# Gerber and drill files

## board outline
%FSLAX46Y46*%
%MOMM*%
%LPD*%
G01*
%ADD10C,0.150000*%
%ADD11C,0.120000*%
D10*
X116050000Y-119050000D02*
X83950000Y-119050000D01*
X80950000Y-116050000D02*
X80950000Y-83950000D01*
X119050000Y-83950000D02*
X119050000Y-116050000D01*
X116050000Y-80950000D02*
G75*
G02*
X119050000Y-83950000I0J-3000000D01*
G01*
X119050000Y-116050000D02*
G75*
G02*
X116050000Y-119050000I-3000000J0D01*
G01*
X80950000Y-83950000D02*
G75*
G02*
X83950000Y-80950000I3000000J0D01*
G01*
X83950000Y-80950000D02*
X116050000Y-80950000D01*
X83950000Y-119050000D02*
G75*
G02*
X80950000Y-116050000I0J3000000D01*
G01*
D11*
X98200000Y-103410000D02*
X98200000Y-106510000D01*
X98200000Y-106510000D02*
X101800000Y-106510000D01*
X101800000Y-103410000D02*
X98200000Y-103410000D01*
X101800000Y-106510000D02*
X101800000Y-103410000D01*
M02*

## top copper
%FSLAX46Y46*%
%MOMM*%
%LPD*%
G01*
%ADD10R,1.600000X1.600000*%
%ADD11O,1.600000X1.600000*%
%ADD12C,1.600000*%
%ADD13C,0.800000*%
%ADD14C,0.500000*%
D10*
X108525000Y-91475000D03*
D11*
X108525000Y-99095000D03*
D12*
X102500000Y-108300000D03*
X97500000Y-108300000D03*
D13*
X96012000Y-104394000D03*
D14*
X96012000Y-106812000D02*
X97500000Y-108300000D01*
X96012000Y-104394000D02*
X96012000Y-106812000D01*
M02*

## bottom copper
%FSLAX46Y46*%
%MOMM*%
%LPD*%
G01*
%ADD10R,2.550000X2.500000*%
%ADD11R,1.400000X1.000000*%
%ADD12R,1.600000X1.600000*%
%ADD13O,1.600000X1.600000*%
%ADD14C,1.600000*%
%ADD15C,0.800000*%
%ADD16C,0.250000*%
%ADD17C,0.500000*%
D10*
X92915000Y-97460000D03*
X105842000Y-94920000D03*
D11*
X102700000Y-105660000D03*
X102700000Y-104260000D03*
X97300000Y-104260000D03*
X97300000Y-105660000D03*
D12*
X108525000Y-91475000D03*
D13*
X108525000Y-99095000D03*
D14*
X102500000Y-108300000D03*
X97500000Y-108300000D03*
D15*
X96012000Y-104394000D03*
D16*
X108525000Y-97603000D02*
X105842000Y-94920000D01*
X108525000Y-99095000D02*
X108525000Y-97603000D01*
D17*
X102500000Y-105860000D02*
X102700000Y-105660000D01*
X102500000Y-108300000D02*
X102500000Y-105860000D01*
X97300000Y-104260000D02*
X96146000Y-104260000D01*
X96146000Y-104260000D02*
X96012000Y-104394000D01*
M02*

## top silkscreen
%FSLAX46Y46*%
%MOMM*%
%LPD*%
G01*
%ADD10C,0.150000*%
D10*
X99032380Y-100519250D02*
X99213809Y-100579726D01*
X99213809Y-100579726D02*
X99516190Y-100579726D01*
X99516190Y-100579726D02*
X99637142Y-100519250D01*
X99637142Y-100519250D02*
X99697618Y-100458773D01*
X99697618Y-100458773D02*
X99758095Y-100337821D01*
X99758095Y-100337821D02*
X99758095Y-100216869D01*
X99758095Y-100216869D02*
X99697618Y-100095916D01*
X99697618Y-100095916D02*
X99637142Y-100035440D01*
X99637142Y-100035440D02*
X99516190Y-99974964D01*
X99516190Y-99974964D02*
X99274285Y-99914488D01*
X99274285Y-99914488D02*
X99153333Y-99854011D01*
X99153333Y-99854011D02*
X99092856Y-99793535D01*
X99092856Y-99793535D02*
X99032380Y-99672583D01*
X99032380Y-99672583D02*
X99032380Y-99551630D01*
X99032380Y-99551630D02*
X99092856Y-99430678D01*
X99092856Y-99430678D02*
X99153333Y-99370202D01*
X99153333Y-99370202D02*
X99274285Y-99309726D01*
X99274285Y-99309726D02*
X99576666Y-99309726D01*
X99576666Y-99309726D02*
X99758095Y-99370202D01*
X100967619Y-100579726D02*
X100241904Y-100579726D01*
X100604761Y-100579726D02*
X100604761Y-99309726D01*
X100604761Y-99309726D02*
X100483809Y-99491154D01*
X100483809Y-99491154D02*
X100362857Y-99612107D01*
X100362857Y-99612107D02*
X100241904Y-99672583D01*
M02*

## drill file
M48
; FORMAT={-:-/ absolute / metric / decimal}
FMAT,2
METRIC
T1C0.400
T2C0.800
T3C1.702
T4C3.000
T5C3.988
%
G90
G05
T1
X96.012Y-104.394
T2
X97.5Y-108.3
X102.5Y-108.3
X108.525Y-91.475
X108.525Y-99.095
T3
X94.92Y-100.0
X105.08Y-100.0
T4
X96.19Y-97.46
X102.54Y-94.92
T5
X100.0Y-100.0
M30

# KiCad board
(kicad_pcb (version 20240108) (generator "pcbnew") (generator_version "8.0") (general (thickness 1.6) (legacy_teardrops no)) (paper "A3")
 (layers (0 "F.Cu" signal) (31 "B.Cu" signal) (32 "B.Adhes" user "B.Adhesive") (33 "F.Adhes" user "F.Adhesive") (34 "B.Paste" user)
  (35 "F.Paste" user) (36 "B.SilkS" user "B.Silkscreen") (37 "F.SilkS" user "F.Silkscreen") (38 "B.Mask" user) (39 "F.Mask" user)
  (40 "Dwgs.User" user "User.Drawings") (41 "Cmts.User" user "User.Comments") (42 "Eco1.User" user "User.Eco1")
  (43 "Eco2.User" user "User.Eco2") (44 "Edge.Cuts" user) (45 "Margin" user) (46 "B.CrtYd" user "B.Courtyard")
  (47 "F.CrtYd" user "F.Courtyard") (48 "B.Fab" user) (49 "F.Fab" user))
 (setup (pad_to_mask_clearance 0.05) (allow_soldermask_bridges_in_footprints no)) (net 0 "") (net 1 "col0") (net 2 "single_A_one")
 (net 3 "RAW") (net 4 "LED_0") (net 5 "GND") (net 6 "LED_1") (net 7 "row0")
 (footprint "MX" (layer "F.Cu") (at 100 100)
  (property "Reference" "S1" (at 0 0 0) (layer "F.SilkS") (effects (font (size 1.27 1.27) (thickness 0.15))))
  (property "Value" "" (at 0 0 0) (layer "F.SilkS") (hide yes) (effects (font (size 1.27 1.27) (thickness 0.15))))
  (pad "" np_thru_hole circle (at -5.08 0) (size 1.7018 1.7018) (drill 1.7018) (layers "*.Cu" "*.Mask"))
  (pad "" np_thru_hole circle (at -3.81 -2.54) (size 3 3) (drill 3) (layers "*.Cu" "*.Mask"))
  (pad "" np_thru_hole circle (at 0 0) (size 3.9878 3.9878) (drill 3.9878) (layers "*.Cu" "*.Mask"))
  (pad "" np_thru_hole circle (at 2.54 -5.08) (size 3 3) (drill 3) (layers "*.Cu" "*.Mask"))
  (pad "" np_thru_hole circle (at 5.08 0) (size 1.7018 1.7018) (drill 1.7018) (layers "*.Cu" "*.Mask"))
  (pad "1" smd rect (at -7.085 -2.54) (size 2.55 2.5) (layers "B.Cu" "B.Paste" "B.Mask") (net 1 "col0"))
  (pad "2" smd rect (at 5.842 -5.08) (size 2.55 2.5) (layers "B.Cu" "B.Paste" "B.Mask") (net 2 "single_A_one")))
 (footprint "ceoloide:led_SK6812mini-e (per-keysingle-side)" (layer "B.Cu") (at 100 104.96)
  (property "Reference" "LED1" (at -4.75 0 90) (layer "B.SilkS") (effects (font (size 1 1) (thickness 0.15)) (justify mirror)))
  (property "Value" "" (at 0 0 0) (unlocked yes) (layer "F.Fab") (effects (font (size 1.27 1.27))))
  (fp_line (start -1.8 -1.55) (end -1.8 1.55) (stroke (width 0.12) (type solid)) (layer "Edge.Cuts"))
  (fp_line (start -1.8 1.55) (end 1.8 1.55) (stroke (width 0.12) (type solid)) (layer "Edge.Cuts"))
  (fp_line (start 1.8 -1.55) (end -1.8 -1.55) (stroke (width 0.12) (type solid)) (layer "Edge.Cuts"))
  (fp_line (start 1.8 1.55) (end 1.8 -1.55) (stroke (width 0.12) (type solid)) (layer "Edge.Cuts"))
  (pad "1" smd rect (at 2.7 0.7) (size 1.4 1) (layers "B.Cu" "B.Paste" "B.Mask") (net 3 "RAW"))
  (pad "2" smd rect (at 2.7 -0.7) (size 1.4 1) (layers "B.Cu" "B.Paste" "B.Mask") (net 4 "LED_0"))
  (pad "3" smd rect (at -2.7 -0.7) (size 1.4 1) (layers "B.Cu" "B.Paste" "B.Mask") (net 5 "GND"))
  (pad "4" smd rect (at -2.7 0.7) (size 1.4 1) (layers "B.Cu" "B.Paste" "B.Mask") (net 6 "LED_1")))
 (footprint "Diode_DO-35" (layer "B.Cu") (at 108.525 91.475 -90)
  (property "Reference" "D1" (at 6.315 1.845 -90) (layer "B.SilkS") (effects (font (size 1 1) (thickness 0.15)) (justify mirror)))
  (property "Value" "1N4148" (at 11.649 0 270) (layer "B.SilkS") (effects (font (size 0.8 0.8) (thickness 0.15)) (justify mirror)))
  (pad "1" thru_hole rect (at 0 0 270) (size 1.6 1.6) (drill 0.8) (layers "*.Cu" "*.Mask") (remove_unused_layers no) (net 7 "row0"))
  (pad "2" thru_hole oval (at 7.62 0 270) (size 1.6 1.6) (drill 0.8) (layers "*.Cu" "*.Mask") (remove_unused_layers no)
   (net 2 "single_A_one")))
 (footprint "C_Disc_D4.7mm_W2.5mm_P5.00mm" (layer "B.Cu") (at 102.5 108.3 180)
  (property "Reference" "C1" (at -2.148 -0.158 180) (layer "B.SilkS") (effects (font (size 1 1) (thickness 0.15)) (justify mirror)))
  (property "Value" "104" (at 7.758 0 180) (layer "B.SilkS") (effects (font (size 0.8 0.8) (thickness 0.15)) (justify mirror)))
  (pad "1" thru_hole circle (at 0 0) (size 1.6 1.6) (drill 0.8) (layers "*.Cu" "*.Mask") (remove_unused_layers no) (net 3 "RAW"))
  (pad "2" thru_hole circle (at 5 0) (size 1.6 1.6) (drill 0.8) (layers "*.Cu" "*.Mask") (remove_unused_layers no) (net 5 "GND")))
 (gr_line (start 116.05 119.05) (end 83.95 119.05) (stroke (width 0.15) (type solid)) (layer "Edge.Cuts"))
 (gr_line (start 80.95 116.05) (end 80.95 83.95) (stroke (width 0.15) (type solid)) (layer "Edge.Cuts"))
 (gr_line (start 119.05 83.95) (end 119.05 116.05) (stroke (width 0.15) (type solid)) (layer "Edge.Cuts"))
 (gr_arc (start 116.05 80.95) (mid 118.17132 81.82868) (end 119.05 83.95) (stroke (width 0.15) (type solid)) (layer "Edge.Cuts"))
 (gr_arc (start 119.05 116.05) (mid 118.17132 118.17132) (end 116.05 119.05) (stroke (width 0.15) (type solid)) (layer "Edge.Cuts"))
 (gr_arc (start 80.95 83.95) (mid 81.82868 81.82868) (end 83.95 80.95) (stroke (width 0.15) (type solid)) (layer "Edge.Cuts"))
 (gr_line (start 83.95 80.95) (end 116.05 80.95) (stroke (width 0.15) (type solid)) (layer "Edge.Cuts"))
 (gr_arc (start 83.95 119.05) (mid 81.82868 118.17132) (end 80.95 116.05) (stroke (width 0.15) (type solid)) (layer "Edge.Cuts"))
 (segment (start 108.525 97.603) (end 105.842 94.92) (width 0.25) (layer "B.Cu") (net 2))
 (segment (start 108.525 99.095) (end 108.525 97.603) (width 0.25) (layer "B.Cu") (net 2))
 (segment (start 102.5 105.86) (end 102.7 105.66) (width 0.5) (layer "B.Cu") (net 3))
 (segment (start 102.5 108.3) (end 102.5 105.86) (width 0.5) (layer "B.Cu") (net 3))
 (segment (start 96.012 106.812) (end 97.5 108.3) (width 0.5) (layer "F.Cu") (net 5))
 (segment (start 96.012 104.394) (end 96.012 106.812) (width 0.5) (layer "F.Cu") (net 5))
 (via (at 96.012 104.394) (size 0.8) (drill 0.4) (layers "F.Cu" "B.Cu") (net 5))
 (segment (start 97.3 104.26) (end 96.146 104.26) (width 0.5) (layer "B.Cu") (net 5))
 (segment (start 96.146 104.26) (end 96.012 104.394) (width 0.5) (layer "B.Cu") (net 5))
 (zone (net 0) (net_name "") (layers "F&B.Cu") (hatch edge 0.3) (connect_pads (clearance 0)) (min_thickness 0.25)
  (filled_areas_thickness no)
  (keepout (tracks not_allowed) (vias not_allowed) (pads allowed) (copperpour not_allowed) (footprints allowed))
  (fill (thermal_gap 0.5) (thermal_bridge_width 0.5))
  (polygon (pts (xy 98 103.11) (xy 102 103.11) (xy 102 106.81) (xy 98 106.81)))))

